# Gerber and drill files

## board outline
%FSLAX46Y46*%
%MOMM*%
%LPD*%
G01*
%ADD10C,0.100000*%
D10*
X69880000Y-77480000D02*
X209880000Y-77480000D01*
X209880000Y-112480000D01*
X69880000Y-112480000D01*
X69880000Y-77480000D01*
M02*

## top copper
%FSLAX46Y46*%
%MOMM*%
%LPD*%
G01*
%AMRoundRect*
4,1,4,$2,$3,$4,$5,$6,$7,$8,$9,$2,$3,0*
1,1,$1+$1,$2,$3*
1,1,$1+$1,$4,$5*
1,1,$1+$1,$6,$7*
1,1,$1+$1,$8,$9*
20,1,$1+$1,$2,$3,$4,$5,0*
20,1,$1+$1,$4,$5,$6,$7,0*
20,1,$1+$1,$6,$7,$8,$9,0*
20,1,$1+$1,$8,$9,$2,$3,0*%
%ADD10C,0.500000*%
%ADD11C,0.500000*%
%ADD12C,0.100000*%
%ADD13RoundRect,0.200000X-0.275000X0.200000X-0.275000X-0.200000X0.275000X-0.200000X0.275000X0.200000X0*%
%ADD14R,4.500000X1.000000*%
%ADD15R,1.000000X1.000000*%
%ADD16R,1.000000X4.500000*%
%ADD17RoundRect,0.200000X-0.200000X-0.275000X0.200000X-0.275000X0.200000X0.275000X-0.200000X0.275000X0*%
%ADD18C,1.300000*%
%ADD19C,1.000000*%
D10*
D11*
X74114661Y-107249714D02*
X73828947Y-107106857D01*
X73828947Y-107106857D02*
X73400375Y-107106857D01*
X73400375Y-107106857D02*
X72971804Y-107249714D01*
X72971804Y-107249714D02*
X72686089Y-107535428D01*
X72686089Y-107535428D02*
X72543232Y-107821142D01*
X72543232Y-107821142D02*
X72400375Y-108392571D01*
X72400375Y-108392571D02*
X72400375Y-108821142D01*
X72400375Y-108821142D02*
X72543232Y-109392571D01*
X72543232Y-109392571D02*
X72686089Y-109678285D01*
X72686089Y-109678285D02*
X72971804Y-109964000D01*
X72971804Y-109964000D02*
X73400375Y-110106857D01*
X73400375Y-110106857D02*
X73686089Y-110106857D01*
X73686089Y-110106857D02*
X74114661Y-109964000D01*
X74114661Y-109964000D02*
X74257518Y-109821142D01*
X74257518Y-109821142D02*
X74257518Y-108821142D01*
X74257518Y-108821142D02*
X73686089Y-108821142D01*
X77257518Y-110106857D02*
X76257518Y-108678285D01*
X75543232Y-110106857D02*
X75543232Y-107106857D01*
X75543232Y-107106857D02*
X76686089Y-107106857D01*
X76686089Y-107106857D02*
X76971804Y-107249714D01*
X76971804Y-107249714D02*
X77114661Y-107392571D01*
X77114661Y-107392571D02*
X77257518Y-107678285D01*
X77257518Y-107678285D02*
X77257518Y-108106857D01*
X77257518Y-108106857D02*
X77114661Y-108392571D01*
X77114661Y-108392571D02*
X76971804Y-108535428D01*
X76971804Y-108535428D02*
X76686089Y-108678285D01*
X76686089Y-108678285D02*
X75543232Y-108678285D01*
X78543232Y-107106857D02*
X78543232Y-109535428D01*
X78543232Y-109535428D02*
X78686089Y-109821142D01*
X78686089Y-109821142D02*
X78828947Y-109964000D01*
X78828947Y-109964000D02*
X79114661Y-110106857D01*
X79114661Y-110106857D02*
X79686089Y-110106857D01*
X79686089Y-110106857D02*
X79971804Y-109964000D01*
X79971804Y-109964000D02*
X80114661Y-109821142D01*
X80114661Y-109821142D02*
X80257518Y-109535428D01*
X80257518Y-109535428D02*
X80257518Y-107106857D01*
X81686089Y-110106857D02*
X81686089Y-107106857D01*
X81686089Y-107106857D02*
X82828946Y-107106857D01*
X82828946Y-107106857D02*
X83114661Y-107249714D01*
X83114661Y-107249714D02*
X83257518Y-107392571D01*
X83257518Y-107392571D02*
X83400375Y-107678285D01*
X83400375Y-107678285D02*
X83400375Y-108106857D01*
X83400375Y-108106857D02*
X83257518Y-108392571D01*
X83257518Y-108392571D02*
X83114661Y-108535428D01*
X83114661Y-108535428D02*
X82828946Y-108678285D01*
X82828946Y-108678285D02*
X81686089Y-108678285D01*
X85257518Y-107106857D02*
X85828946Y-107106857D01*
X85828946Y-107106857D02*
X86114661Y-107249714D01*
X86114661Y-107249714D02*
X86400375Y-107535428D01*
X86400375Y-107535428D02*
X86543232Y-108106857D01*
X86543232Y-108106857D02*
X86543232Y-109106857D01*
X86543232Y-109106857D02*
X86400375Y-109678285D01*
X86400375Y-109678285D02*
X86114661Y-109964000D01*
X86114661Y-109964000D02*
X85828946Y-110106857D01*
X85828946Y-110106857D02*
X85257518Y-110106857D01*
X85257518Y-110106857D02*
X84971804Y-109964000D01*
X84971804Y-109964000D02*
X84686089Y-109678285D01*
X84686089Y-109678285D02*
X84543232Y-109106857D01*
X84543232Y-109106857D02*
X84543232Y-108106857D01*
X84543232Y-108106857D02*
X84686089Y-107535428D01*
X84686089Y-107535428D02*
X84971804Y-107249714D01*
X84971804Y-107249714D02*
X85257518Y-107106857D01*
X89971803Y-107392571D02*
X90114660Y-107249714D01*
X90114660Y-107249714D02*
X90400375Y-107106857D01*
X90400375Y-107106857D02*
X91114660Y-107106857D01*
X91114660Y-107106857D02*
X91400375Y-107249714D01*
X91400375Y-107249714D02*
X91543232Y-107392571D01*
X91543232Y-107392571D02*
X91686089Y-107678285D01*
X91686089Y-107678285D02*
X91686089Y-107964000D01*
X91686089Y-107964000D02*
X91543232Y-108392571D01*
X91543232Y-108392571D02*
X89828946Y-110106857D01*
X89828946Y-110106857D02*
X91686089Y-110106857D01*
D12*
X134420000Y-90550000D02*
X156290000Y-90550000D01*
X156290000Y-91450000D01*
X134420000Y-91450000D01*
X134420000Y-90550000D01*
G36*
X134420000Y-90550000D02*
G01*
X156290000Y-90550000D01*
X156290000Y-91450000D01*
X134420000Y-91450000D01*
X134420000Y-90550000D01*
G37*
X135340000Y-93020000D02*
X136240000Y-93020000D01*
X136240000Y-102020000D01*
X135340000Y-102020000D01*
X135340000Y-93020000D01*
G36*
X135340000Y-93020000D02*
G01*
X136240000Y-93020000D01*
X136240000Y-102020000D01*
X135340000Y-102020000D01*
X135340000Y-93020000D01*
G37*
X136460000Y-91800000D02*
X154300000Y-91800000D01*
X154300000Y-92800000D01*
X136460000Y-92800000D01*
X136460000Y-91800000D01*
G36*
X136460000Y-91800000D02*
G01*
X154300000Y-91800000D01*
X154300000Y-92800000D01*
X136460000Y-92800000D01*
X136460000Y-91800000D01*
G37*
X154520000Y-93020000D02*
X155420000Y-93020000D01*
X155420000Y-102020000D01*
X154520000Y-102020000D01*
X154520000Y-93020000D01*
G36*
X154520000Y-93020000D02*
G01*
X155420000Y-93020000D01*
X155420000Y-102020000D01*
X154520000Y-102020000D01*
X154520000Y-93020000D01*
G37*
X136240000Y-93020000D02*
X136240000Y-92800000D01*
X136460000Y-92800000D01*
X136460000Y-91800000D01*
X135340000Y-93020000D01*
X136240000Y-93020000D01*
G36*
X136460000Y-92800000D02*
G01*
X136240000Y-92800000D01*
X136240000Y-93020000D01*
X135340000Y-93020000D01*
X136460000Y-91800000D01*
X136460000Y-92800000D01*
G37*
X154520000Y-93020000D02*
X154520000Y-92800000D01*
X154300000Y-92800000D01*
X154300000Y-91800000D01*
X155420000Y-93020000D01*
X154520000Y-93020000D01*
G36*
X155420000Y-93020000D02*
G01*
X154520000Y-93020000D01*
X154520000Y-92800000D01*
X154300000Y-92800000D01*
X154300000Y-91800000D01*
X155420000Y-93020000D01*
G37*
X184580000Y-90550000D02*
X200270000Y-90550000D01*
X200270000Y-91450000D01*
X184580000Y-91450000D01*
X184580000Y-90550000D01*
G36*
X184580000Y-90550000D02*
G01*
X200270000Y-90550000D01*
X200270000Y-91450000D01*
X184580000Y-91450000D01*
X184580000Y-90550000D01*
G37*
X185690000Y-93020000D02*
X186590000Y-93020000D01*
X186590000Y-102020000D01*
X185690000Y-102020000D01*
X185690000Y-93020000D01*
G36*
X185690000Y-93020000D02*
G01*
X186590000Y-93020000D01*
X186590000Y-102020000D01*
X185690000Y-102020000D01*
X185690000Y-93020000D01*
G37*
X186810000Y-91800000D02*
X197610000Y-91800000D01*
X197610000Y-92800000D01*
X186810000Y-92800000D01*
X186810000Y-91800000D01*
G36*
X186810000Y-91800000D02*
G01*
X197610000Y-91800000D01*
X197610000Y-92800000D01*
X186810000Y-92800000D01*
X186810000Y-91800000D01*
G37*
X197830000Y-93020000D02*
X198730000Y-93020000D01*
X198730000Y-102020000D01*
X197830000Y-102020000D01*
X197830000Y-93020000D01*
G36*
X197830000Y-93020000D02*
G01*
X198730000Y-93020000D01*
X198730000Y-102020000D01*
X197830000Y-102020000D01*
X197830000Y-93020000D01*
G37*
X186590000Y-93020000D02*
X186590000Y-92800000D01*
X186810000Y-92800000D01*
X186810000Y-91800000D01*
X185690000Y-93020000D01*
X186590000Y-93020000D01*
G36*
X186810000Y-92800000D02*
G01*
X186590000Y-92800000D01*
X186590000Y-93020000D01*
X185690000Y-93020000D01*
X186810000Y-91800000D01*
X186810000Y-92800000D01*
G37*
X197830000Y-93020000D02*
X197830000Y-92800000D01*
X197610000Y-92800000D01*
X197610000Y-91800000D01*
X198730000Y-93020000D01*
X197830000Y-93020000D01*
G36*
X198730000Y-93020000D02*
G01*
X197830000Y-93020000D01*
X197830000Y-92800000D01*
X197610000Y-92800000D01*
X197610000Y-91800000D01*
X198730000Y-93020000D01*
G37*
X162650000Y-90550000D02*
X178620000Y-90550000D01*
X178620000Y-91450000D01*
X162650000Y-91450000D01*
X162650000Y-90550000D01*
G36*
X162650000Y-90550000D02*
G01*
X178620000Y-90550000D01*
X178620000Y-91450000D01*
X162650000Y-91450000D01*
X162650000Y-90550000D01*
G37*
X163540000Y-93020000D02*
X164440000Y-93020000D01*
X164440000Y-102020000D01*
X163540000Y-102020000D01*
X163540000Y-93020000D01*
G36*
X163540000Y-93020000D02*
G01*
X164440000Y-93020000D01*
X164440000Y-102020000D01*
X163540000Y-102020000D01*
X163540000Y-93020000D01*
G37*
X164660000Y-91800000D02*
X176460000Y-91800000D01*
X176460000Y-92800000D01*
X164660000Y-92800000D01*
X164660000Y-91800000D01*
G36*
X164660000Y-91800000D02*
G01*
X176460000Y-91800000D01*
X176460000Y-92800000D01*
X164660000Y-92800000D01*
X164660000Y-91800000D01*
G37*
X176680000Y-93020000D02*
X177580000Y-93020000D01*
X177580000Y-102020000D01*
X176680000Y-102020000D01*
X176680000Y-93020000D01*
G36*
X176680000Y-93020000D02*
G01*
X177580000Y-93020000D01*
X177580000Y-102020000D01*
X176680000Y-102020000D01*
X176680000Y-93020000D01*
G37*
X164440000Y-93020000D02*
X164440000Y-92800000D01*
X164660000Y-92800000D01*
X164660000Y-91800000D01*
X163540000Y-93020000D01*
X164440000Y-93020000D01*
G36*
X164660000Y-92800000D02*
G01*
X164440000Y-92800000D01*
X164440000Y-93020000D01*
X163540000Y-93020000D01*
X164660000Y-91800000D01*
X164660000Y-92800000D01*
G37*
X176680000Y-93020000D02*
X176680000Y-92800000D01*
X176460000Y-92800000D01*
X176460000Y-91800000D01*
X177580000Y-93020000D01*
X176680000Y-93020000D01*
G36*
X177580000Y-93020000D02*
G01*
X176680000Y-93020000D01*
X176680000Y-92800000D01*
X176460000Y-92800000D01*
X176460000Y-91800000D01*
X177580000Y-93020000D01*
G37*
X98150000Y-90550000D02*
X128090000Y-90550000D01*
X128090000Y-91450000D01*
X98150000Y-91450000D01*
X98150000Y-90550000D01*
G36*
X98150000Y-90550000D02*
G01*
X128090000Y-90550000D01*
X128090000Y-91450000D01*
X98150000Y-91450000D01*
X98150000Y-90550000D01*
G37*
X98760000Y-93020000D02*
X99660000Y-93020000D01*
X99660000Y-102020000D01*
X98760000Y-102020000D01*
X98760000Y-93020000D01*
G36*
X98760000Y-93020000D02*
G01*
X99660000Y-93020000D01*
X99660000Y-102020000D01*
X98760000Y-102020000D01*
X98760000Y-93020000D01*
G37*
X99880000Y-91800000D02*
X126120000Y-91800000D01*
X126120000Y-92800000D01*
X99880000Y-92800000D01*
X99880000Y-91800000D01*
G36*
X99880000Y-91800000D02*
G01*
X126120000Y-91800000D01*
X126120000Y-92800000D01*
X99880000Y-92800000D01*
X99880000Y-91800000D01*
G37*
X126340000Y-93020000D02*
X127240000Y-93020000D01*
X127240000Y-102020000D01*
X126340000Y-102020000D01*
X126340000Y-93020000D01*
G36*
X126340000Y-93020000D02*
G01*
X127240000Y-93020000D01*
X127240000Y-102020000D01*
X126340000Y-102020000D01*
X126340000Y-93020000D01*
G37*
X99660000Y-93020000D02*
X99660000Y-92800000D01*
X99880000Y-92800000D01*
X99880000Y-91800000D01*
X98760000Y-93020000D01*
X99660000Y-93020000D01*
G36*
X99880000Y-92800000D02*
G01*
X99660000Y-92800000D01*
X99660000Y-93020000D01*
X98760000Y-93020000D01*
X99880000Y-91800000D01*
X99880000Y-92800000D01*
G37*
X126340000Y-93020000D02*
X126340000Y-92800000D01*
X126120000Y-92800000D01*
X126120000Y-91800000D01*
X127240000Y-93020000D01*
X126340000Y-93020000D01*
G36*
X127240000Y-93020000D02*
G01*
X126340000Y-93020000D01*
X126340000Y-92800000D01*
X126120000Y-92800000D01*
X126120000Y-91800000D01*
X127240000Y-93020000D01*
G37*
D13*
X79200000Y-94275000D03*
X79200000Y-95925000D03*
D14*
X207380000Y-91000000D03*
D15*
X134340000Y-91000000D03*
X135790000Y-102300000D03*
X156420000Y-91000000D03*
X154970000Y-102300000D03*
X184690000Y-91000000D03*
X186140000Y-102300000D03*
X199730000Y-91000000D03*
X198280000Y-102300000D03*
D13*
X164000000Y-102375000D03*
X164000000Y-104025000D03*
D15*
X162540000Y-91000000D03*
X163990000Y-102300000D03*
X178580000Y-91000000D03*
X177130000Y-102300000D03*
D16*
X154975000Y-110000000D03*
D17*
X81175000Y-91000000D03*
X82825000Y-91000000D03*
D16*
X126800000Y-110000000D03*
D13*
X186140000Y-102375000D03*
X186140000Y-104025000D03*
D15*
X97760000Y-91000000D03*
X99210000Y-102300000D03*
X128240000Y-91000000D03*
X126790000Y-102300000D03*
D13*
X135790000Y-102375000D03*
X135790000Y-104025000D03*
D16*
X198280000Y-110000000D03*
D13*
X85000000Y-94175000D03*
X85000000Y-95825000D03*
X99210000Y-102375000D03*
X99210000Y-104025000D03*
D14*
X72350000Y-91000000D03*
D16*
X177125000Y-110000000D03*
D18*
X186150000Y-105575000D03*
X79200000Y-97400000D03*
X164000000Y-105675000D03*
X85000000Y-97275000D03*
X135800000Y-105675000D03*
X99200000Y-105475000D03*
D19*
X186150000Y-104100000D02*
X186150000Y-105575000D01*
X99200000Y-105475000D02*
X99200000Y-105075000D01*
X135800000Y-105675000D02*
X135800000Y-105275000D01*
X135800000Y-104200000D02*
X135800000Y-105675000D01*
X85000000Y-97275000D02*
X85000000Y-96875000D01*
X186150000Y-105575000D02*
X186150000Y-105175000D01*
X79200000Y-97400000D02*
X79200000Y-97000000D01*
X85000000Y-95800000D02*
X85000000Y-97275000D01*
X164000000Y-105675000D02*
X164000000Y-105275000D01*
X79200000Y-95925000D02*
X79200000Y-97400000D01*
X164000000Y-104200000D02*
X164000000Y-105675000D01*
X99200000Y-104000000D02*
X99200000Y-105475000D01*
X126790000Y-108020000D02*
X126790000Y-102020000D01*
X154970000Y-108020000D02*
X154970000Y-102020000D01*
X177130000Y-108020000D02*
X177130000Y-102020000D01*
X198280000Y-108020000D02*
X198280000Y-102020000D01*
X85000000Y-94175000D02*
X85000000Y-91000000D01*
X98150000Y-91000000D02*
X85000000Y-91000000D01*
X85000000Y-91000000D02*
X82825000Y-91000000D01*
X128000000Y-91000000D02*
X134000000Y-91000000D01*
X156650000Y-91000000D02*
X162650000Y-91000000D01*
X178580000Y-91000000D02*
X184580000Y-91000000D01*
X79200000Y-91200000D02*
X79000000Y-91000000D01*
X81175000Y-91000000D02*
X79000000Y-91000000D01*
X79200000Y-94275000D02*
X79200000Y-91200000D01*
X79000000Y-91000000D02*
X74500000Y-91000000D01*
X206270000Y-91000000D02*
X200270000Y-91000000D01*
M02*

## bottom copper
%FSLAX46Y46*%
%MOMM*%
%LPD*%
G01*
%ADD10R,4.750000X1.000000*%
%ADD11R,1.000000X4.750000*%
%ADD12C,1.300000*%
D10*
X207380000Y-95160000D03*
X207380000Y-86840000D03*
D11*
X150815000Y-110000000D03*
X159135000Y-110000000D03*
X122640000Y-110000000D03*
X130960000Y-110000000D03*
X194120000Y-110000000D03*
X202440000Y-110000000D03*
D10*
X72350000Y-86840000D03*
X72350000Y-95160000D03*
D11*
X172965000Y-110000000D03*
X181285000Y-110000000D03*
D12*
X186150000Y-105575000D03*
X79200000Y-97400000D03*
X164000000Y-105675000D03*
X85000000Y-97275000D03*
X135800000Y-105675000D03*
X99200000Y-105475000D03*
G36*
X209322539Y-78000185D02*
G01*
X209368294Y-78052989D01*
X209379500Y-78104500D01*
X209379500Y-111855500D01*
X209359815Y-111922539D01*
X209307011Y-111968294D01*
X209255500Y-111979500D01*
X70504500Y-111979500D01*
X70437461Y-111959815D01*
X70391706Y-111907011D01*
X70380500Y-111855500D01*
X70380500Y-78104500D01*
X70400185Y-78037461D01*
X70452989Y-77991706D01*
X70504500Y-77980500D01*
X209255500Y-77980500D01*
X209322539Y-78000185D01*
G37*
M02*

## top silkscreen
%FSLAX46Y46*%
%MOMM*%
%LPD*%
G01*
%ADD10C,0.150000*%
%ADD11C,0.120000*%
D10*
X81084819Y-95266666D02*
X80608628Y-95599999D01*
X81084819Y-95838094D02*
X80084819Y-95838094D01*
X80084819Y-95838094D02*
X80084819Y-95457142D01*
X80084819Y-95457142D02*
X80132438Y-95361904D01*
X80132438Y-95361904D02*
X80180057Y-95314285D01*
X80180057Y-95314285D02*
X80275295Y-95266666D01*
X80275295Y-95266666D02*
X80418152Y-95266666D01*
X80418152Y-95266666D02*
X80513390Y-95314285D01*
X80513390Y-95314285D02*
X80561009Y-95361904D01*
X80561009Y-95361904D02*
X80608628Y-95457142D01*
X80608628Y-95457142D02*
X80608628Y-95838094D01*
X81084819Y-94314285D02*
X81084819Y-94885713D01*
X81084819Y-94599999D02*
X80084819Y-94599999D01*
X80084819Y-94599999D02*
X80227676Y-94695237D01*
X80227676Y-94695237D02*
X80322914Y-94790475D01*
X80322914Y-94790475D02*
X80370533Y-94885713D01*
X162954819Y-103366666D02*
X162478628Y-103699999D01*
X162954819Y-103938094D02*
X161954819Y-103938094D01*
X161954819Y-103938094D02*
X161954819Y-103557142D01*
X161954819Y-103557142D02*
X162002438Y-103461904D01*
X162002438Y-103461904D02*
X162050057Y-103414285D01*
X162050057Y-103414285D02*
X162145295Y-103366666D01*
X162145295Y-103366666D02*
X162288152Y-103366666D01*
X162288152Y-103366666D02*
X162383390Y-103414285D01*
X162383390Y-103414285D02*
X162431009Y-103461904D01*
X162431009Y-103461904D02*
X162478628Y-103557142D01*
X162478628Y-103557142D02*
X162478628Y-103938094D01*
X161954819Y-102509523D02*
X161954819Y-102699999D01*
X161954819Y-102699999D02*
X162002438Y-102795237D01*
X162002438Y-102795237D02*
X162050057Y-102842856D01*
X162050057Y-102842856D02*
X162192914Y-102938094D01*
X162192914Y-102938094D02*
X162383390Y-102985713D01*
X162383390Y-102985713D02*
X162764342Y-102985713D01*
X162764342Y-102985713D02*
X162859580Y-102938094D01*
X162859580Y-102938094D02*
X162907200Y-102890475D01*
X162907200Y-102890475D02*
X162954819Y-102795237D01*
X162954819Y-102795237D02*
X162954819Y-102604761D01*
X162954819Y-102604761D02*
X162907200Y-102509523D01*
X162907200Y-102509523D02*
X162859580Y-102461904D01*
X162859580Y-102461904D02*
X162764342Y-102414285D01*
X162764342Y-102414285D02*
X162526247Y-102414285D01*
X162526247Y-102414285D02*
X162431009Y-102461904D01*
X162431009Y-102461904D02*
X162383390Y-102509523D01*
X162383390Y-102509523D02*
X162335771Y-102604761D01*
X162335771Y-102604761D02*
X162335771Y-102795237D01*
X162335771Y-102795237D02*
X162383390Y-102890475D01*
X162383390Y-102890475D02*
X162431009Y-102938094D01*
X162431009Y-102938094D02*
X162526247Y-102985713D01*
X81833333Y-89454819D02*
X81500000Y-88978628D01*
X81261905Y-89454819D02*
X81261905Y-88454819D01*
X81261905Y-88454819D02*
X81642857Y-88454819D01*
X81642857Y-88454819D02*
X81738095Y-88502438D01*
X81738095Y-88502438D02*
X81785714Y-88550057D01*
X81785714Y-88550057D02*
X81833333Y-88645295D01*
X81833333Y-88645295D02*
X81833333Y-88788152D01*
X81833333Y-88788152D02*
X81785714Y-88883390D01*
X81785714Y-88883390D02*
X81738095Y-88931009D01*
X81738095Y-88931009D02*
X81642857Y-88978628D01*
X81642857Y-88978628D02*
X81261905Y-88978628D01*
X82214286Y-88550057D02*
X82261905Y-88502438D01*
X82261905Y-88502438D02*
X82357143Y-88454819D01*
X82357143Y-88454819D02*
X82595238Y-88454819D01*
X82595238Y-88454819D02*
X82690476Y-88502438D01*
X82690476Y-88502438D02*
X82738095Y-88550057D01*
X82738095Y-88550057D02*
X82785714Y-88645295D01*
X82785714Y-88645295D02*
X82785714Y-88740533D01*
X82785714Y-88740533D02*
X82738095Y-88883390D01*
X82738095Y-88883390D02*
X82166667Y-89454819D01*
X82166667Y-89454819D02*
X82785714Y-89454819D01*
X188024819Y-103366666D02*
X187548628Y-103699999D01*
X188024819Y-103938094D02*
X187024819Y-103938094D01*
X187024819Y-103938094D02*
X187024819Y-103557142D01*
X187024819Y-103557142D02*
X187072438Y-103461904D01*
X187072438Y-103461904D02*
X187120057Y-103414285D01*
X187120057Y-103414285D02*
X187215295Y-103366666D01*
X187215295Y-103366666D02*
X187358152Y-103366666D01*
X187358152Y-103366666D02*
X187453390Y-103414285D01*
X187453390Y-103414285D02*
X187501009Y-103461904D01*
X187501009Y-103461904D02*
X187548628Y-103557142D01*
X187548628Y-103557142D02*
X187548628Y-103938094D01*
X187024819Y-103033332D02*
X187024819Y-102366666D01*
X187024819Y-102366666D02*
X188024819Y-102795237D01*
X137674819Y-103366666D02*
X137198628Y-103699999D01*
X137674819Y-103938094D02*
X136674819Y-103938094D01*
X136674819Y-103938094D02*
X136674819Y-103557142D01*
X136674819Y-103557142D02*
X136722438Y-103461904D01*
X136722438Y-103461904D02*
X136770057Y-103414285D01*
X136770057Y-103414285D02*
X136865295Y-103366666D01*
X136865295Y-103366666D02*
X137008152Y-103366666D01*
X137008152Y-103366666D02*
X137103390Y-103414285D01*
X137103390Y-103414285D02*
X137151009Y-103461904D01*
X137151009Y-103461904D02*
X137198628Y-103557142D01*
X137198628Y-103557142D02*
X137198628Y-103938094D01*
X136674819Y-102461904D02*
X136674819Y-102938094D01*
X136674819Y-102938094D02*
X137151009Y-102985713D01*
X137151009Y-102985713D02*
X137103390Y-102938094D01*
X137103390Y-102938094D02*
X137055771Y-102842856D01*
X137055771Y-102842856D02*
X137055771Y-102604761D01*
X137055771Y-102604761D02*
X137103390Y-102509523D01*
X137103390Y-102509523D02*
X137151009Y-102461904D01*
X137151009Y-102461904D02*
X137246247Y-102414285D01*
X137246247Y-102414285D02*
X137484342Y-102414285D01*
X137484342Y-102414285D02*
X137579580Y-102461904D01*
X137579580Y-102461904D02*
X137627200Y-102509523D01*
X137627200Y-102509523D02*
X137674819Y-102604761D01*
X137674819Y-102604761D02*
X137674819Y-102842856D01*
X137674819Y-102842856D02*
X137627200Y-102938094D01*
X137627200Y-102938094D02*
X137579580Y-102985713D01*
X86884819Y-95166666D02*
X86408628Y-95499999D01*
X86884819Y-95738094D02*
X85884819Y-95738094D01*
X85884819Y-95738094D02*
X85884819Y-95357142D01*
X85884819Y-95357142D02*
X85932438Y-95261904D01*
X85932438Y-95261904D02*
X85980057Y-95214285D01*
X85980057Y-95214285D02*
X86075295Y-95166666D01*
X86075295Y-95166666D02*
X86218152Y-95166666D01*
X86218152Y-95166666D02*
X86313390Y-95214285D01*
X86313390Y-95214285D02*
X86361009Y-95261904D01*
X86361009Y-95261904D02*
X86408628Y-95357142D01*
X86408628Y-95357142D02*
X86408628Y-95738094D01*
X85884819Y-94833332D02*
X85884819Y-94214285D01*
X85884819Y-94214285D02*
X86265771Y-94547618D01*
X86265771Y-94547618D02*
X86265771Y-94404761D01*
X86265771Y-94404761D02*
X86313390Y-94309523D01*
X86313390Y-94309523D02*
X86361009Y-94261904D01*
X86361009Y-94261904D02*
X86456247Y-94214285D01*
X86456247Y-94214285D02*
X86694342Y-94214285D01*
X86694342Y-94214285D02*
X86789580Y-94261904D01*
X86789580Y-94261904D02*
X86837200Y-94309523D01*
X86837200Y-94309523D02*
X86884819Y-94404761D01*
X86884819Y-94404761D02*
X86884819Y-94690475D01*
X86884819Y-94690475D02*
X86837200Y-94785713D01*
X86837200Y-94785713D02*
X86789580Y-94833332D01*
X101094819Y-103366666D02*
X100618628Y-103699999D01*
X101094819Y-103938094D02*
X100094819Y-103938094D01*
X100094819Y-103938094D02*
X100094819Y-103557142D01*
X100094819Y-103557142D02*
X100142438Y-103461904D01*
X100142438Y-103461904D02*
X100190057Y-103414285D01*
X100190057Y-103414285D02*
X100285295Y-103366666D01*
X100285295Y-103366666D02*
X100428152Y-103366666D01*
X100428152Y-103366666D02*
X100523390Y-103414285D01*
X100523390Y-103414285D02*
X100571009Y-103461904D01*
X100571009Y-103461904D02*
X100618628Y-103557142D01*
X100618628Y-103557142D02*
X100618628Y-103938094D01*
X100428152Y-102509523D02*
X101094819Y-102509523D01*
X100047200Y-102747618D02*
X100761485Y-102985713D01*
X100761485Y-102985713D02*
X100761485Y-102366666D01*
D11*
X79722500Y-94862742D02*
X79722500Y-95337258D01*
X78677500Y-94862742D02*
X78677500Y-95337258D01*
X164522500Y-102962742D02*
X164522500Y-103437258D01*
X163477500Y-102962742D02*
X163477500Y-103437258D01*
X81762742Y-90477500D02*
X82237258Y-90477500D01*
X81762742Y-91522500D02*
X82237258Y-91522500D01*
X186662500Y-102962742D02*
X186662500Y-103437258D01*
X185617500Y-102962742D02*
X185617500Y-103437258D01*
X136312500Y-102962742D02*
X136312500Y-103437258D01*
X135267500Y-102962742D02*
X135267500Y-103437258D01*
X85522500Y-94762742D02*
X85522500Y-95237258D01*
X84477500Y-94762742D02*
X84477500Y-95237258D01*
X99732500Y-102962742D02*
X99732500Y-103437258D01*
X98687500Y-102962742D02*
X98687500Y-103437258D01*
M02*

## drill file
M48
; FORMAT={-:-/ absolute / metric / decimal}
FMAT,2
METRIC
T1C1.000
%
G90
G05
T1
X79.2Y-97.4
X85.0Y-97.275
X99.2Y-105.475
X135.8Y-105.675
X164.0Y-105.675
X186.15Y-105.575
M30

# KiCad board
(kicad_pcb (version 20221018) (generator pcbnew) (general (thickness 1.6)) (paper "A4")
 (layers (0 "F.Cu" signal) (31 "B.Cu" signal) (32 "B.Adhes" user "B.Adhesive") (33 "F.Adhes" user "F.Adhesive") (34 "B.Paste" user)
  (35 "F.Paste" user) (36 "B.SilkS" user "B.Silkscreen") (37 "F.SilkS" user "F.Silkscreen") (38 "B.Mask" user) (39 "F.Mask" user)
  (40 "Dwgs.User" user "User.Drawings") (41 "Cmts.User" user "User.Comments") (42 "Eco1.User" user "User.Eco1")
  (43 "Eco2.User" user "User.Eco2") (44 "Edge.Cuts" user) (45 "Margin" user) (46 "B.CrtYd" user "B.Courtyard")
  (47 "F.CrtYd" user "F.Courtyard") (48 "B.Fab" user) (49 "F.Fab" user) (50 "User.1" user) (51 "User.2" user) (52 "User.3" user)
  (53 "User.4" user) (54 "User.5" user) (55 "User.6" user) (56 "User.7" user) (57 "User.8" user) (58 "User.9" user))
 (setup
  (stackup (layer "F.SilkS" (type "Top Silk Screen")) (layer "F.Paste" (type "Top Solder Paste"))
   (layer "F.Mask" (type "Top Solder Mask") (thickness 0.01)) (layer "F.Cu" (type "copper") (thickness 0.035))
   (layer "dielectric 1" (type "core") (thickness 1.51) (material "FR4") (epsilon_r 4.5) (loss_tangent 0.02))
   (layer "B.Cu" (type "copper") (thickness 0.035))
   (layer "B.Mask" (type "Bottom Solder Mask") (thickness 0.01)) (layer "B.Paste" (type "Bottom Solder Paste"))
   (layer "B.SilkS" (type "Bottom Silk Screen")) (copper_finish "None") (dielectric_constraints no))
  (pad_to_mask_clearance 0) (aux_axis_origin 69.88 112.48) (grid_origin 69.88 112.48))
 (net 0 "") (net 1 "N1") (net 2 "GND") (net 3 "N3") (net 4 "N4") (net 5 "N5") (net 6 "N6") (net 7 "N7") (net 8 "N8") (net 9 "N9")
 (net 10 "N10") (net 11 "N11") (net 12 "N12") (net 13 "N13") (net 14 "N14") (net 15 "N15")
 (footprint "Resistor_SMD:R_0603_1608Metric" (layer "F.Cu") (at 79.2 95.1 -90)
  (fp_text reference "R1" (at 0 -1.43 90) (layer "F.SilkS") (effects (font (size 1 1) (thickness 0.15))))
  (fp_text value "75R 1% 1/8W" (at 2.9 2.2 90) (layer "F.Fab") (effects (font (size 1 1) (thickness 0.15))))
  (fp_line (start -0.237258 -0.5225) (end 0.237258 -0.5225) (stroke (width 0.12) (type solid)) (layer "F.SilkS"))
  (fp_line (start -0.237258 0.5225) (end 0.237258 0.5225) (stroke (width 0.12) (type solid)) (layer "F.SilkS"))
  (pad "1" smd roundrect (at -0.825 0 270) (size 0.8 0.95) (layers "F.Cu" "F.Paste" "F.Mask") (roundrect_rratio 0.25) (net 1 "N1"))
  (pad "2" smd roundrect (at 0.825 0 270) (size 0.8 0.95) (layers "F.Cu" "F.Paste" "F.Mask") (roundrect_rratio 0.25) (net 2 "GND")))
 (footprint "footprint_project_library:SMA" (layer "F.Cu") (at 207.38 91 180)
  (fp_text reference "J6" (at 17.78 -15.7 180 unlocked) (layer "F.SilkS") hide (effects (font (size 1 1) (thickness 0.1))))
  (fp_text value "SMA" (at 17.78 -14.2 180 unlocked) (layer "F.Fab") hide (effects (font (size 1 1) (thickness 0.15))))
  (pad "1" smd rect (at 0 0 180) (size 4.5 1) (layers "F.Cu") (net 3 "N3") (thermal_bridge_angle 45))
  (pad "2" smd rect (at 0 -4.16 180) (size 4.75 1) (layers "B.Cu") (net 2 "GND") (thermal_bridge_angle 45))
  (pad "2" smd rect (at 0 4.16 180) (size 4.75 1) (layers "B.Cu") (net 2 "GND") (thermal_bridge_angle 45)))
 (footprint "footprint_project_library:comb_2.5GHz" (layer "F.Cu") (at 145.38 91)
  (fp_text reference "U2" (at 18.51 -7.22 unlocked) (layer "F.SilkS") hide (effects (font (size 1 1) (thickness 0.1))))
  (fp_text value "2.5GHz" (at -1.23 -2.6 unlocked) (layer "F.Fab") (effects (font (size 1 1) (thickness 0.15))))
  (fp_rect (start -10.96 -0.45) (end 10.91 0.45) (stroke (width 0.1) (type solid)) (fill solid) (layer "F.Cu"))
  (fp_rect (start -10.04 2.02) (end -9.14 11.02) (stroke (width 0.1) (type solid)) (fill solid) (layer "F.Cu"))
  (fp_rect (start -8.92 0.8) (end 8.92 1.8) (stroke (width 0.1) (type solid)) (fill solid) (layer "F.Cu"))
  (fp_rect (start 10.04 2.02) (end 9.14 11.02) (stroke (width 0.1) (type solid)) (fill solid) (layer "F.Cu"))
  (fp_poly
   (pts (xy -9.14 2.02) (xy -9.14 1.8) (xy -8.92 1.8) (xy -8.92 0.8) (xy -10.04 2.02)) (stroke (width 0.1) (type solid)) (fill solid)
   (layer "F.Cu"))
  (fp_poly
   (pts (xy 9.14 2.02) (xy 9.14 1.8) (xy 8.92 1.8) (xy 8.92 0.8) (xy 10.04 2.02)) (stroke (width 0.1) (type solid)) (fill solid)
   (layer "F.Cu"))
  (pad "1" smd rect (at -11.04 0) (size 1 1) (layers "F.Cu") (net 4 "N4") (thermal_bridge_angle 45))
  (pad "2" smd rect (at -9.59 11.3) (size 1 1) (layers "F.Cu") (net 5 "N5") (thermal_bridge_angle 45))
  (pad "3" smd rect (at 11.04 0) (size 1 1) (layers "F.Cu") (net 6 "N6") (thermal_bridge_angle 45))
  (pad "4" smd rect (at 9.59 11.3) (size 1 1) (layers "F.Cu") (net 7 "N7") (thermal_bridge_angle 45)))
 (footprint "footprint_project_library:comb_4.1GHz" (layer "F.Cu") (at 192.21 91)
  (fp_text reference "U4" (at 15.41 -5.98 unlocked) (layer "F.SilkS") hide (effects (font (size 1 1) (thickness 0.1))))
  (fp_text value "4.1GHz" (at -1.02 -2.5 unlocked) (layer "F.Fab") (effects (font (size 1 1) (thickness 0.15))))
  (fp_rect (start -7.63 -0.45) (end 8.06 0.45) (stroke (width 0.1) (type solid)) (fill solid) (layer "F.Cu"))
  (fp_rect (start -6.52 2.02) (end -5.62 11.02) (stroke (width 0.1) (type solid)) (fill solid) (layer "F.Cu"))
  (fp_rect (start -5.4 0.8) (end 5.4 1.8) (stroke (width 0.1) (type solid)) (fill solid) (layer "F.Cu"))
  (fp_rect (start 6.52 2.02) (end 5.62 11.02) (stroke (width 0.1) (type solid)) (fill solid) (layer "F.Cu"))
  (fp_poly
   (pts (xy -5.62 2.02) (xy -5.62 1.8) (xy -5.4 1.8) (xy -5.4 0.8) (xy -6.52 2.02)) (stroke (width 0.1) (type solid)) (fill solid)
   (layer "F.Cu"))
  (fp_poly
   (pts (xy 5.62 2.02) (xy 5.62 1.8) (xy 5.4 1.8) (xy 5.4 0.8) (xy 6.52 2.02)) (stroke (width 0.1) (type solid)) (fill solid) (layer "F.Cu"))
  (pad "1" smd rect (at -7.52 0) (size 1 1) (layers "F.Cu") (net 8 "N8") (thermal_bridge_angle 45))
  (pad "2" smd rect (at -6.07 11.3) (size 1 1) (layers "F.Cu") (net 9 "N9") (thermal_bridge_angle 45))
  (pad "3" smd rect (at 7.52 0) (size 1 1) (layers "F.Cu") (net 3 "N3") (thermal_bridge_angle 45))
  (pad "4" smd rect (at 6.07 11.3) (size 1 1) (layers "F.Cu") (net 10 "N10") (thermal_bridge_angle 45)))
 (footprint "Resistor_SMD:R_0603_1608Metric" (layer "F.Cu") (at 164 103.2 -90)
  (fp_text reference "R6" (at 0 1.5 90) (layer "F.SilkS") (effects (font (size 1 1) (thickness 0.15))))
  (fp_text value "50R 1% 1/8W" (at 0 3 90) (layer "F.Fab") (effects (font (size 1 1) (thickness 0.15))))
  (fp_line (start -0.237258 -0.5225) (end 0.237258 -0.5225) (stroke (width 0.12) (type solid)) (layer "F.SilkS"))
  (fp_line (start -0.237258 0.5225) (end 0.237258 0.5225) (stroke (width 0.12) (type solid)) (layer "F.SilkS"))
  (pad "1" smd roundrect (at -0.825 0 270) (size 0.8 0.95) (layers "F.Cu" "F.Paste" "F.Mask") (roundrect_rratio 0.25) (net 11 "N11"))
  (pad "2" smd roundrect (at 0.825 0 270) (size 0.8 0.95) (layers "F.Cu" "F.Paste" "F.Mask") (roundrect_rratio 0.25) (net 2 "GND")))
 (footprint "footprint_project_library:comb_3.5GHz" (layer "F.Cu") (at 170.56 91)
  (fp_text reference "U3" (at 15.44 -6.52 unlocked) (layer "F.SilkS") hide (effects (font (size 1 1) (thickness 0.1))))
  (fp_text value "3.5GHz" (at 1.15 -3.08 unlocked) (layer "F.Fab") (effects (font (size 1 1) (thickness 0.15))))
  (fp_rect (start -7.91 -0.45) (end 8.06 0.45) (stroke (width 0.1) (type solid)) (fill solid) (layer "F.Cu"))
  (fp_rect (start -7.02 2.02) (end -6.12 11.02) (stroke (width 0.1) (type solid)) (fill solid) (layer "F.Cu"))
  (fp_rect (start -5.9 0.8) (end 5.9 1.8) (stroke (width 0.1) (type solid)) (fill solid) (layer "F.Cu"))
  (fp_rect (start 7.02 2.02) (end 6.12 11.02) (stroke (width 0.1) (type solid)) (fill solid) (layer "F.Cu"))
  (fp_poly
   (pts (xy -6.12 2.02) (xy -6.12 1.8) (xy -5.9 1.8) (xy -5.9 0.8) (xy -7.02 2.02)) (stroke (width 0.1) (type solid)) (fill solid)
   (layer "F.Cu"))
  (fp_poly
   (pts (xy 6.12 2.02) (xy 6.12 1.8) (xy 5.9 1.8) (xy 5.9 0.8) (xy 7.02 2.02)) (stroke (width 0.1) (type solid)) (fill solid) (layer "F.Cu"))
  (pad "1" smd rect (at -8.02 0) (size 1 1) (layers "F.Cu") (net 6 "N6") (thermal_bridge_angle 45))
  (pad "2" smd rect (at -6.57 11.3) (size 1 1) (layers "F.Cu") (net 11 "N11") (thermal_bridge_angle 45))
  (pad "3" smd rect (at 8.02 0) (size 1 1) (layers "F.Cu") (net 8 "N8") (thermal_bridge_angle 45))
  (pad "4" smd rect (at 6.57 11.3) (size 1 1) (layers "F.Cu") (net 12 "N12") (thermal_bridge_angle 45)))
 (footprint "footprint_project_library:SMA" (layer "F.Cu") (at 154.975 110 90)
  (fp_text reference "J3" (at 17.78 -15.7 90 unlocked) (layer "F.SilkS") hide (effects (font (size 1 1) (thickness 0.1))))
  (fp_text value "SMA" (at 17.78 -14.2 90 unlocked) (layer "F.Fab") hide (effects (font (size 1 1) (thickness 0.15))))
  (pad "1" smd rect (at 0 0 90) (size 4.5 1) (layers "F.Cu") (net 7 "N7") (thermal_bridge_angle 45))
  (pad "2" smd rect (at 0 -4.16 90) (size 4.75 1) (layers "B.Cu") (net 2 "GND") (thermal_bridge_angle 45))
  (pad "2" smd rect (at 0 4.16 90) (size 4.75 1) (layers "B.Cu") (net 2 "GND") (thermal_bridge_angle 45)))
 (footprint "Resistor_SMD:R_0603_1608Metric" (layer "F.Cu") (at 82 91)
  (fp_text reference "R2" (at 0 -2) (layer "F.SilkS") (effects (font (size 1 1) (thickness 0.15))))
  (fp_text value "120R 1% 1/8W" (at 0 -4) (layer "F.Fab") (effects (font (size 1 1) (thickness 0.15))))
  (fp_line (start -0.237258 -0.5225) (end 0.237258 -0.5225) (stroke (width 0.12) (type solid)) (layer "F.SilkS"))
  (fp_line (start -0.237258 0.5225) (end 0.237258 0.5225) (stroke (width 0.12) (type solid)) (layer "F.SilkS"))
  (pad "1" smd roundrect (at -0.825 0) (size 0.8 0.95) (layers "F.Cu" "F.Paste" "F.Mask") (roundrect_rratio 0.25) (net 1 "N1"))
  (pad "2" smd roundrect (at 0.825 0) (size 0.8 0.95) (layers "F.Cu" "F.Paste" "F.Mask") (roundrect_rratio 0.25) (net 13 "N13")))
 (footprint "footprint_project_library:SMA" (layer "F.Cu") (at 126.8 110 90)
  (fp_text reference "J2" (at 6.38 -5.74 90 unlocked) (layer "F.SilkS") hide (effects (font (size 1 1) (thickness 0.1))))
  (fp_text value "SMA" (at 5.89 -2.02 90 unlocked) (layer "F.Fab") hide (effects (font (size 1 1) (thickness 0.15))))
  (pad "1" smd rect (at 0 0 90) (size 4.5 1) (layers "F.Cu") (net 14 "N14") (thermal_bridge_angle 45))
  (pad "2" smd rect (at 0 -4.16 90) (size 4.75 1) (layers "B.Cu") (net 2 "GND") (thermal_bridge_angle 45))
  (pad "2" smd rect (at 0 4.16 90) (size 4.75 1) (layers "B.Cu") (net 2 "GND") (thermal_bridge_angle 45)))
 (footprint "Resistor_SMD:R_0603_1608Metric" (layer "F.Cu") (at 186.14 103.2 -90)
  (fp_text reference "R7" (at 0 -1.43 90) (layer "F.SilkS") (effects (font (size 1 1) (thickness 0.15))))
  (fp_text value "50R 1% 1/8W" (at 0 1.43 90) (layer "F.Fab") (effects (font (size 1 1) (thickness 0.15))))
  (fp_line (start -0.237258 -0.5225) (end 0.237258 -0.5225) (stroke (width 0.12) (type solid)) (layer "F.SilkS"))
  (fp_line (start -0.237258 0.5225) (end 0.237258 0.5225) (stroke (width 0.12) (type solid)) (layer "F.SilkS"))
  (pad "1" smd roundrect (at -0.825 0 270) (size 0.8 0.95) (layers "F.Cu" "F.Paste" "F.Mask") (roundrect_rratio 0.25) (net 9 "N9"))
  (pad "2" smd roundrect (at 0.825 0 270) (size 0.8 0.95) (layers "F.Cu" "F.Paste" "F.Mask") (roundrect_rratio 0.25) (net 2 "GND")))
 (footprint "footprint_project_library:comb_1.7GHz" (layer "F.Cu") (at 113 91)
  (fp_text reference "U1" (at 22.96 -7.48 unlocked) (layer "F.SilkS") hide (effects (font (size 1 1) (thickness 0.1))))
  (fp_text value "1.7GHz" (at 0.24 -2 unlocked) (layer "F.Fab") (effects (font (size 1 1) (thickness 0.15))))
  (fp_rect (start -14.85 -0.45) (end 15.09 0.45) (stroke (width 0.1) (type solid)) (fill solid) (layer "F.Cu"))
  (fp_rect (start -14.24 2.02) (end -13.34 11.02) (stroke (width 0.1) (type solid)) (fill solid) (layer "F.Cu"))
  (fp_rect (start -13.12 0.8) (end 13.12 1.8) (stroke (width 0.1) (type solid)) (fill solid) (layer "F.Cu"))
  (fp_rect (start 14.24 2.02) (end 13.34 11.02) (stroke (width 0.1) (type solid)) (fill solid) (layer "F.Cu"))
  (fp_poly
   (pts (xy -13.34 2.02) (xy -13.34 1.8) (xy -13.12 1.8) (xy -13.12 0.8) (xy -14.24 2.02)) (stroke (width 0.1) (type solid)) (fill solid)
   (layer "F.Cu"))
  (fp_poly
   (pts (xy 13.34 2.02) (xy 13.34 1.8) (xy 13.12 1.8) (xy 13.12 0.8) (xy 14.24 2.02)) (stroke (width 0.1) (type solid)) (fill solid)
   (layer "F.Cu"))
  (pad "1" smd rect (at -15.24 0) (size 1 1) (layers "F.Cu") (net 13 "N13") (thermal_bridge_angle 45))
  (pad "2" smd rect (at -13.79 11.3) (size 1 1) (layers "F.Cu") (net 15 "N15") (thermal_bridge_angle 45))
  (pad "3" smd rect (at 15.24 0) (size 1 1) (layers "F.Cu") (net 4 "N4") (thermal_bridge_angle 45))
  (pad "4" smd rect (at 13.79 11.3) (size 1 1) (layers "F.Cu") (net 14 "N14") (thermal_bridge_angle 45)))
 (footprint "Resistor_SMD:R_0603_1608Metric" (layer "F.Cu") (at 135.79 103.2 -90)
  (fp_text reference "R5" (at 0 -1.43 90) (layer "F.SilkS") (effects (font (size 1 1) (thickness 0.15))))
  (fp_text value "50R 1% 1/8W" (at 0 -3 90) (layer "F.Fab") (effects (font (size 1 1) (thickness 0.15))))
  (fp_line (start -0.237258 -0.5225) (end 0.237258 -0.5225) (stroke (width 0.12) (type solid)) (layer "F.SilkS"))
  (fp_line (start -0.237258 0.5225) (end 0.237258 0.5225) (stroke (width 0.12) (type solid)) (layer "F.SilkS"))
  (pad "1" smd roundrect (at -0.825 0 270) (size 0.8 0.95) (layers "F.Cu" "F.Paste" "F.Mask") (roundrect_rratio 0.25) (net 5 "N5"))
  (pad "2" smd roundrect (at 0.825 0 270) (size 0.8 0.95) (layers "F.Cu" "F.Paste" "F.Mask") (roundrect_rratio 0.25) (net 2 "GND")))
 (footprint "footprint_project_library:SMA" (layer "F.Cu") (at 198.28 110 90)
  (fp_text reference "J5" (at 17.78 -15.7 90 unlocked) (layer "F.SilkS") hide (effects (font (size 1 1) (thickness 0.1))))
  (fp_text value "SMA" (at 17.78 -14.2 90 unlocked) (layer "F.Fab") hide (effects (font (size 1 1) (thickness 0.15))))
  (pad "1" smd rect (at 0 0 90) (size 4.5 1) (layers "F.Cu") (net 10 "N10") (thermal_bridge_angle 45))
  (pad "2" smd rect (at 0 -4.16 90) (size 4.75 1) (layers "B.Cu") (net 2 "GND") (thermal_bridge_angle 45))
  (pad "2" smd rect (at 0 4.16 90) (size 4.75 1) (layers "B.Cu") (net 2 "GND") (thermal_bridge_angle 45)))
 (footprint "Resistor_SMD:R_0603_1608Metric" (layer "F.Cu") (at 85 95 -90)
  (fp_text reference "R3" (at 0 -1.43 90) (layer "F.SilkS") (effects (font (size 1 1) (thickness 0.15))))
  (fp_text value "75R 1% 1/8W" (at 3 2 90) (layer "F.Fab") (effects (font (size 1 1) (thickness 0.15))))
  (fp_line (start -0.237258 -0.5225) (end 0.237258 -0.5225) (stroke (width 0.12) (type solid)) (layer "F.SilkS"))
  (fp_line (start -0.237258 0.5225) (end 0.237258 0.5225) (stroke (width 0.12) (type solid)) (layer "F.SilkS"))
  (pad "1" smd roundrect (at -0.825 0 270) (size 0.8 0.95) (layers "F.Cu" "F.Paste" "F.Mask") (roundrect_rratio 0.25) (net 13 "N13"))
  (pad "2" smd roundrect (at 0.825 0 270) (size 0.8 0.95) (layers "F.Cu" "F.Paste" "F.Mask") (roundrect_rratio 0.25) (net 2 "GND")))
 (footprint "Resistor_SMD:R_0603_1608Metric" (layer "F.Cu") (at 99.21 103.2 -90)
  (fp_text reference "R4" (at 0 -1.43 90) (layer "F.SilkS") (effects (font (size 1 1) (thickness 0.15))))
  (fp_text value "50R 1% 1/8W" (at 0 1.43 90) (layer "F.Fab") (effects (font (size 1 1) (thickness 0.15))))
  (fp_line (start -0.237258 -0.5225) (end 0.237258 -0.5225) (stroke (width 0.12) (type solid)) (layer "F.SilkS"))
  (fp_line (start -0.237258 0.5225) (end 0.237258 0.5225) (stroke (width 0.12) (type solid)) (layer "F.SilkS"))
  (pad "1" smd roundrect (at -0.825 0 270) (size 0.8 0.95) (layers "F.Cu" "F.Paste" "F.Mask") (roundrect_rratio 0.25) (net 15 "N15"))
  (pad "2" smd roundrect (at 0.825 0 270) (size 0.8 0.95) (layers "F.Cu" "F.Paste" "F.Mask") (roundrect_rratio 0.25) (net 2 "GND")))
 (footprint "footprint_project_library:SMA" (layer "F.Cu") (at 72.35 91)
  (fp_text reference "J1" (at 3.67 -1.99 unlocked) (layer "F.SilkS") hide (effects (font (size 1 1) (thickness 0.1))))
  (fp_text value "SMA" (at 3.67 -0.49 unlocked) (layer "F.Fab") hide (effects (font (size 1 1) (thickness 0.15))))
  (pad "1" smd rect (at 0 0) (size 4.5 1) (layers "F.Cu") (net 1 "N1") (thermal_bridge_angle 45))
  (pad "2" smd rect (at 0 -4.16) (size 4.75 1) (layers "B.Cu") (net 2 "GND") (thermal_bridge_angle 45))
  (pad "2" smd rect (at 0 4.16) (size 4.75 1) (layers "B.Cu") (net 2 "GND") (thermal_bridge_angle 45)))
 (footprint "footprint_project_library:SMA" (layer "F.Cu") (at 177.125 110 90)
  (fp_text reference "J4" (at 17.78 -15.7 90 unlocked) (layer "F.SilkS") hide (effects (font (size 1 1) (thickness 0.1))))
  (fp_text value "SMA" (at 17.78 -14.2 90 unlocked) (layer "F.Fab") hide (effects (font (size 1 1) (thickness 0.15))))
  (pad "1" smd rect (at 0 0 90) (size 4.5 1) (layers "F.Cu") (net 12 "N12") (thermal_bridge_angle 45))
  (pad "2" smd rect (at 0 -4.16 90) (size 4.75 1) (layers "B.Cu") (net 2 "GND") (thermal_bridge_angle 45))
  (pad "2" smd rect (at 0 4.16 90) (size 4.75 1) (layers "B.Cu") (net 2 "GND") (thermal_bridge_angle 45)))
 (gr_rect (start 69.88 77.48) (end 209.88 112.48) (stroke (width 0.1) (type default)) (fill none) (layer "Edge.Cuts"))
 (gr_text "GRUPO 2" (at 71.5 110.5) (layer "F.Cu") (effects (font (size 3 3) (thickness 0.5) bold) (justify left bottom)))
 (segment (start 186.15 104.1) (end 186.15 105.575) (width 1) (layer "F.Cu") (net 2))
 (segment (start 99.2 105.475) (end 99.2 105.075) (width 1) (layer "F.Cu") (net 2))
 (segment (start 135.8 105.675) (end 135.8 105.275) (width 1) (layer "F.Cu") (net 2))
 (segment (start 135.8 104.2) (end 135.8 105.675) (width 1) (layer "F.Cu") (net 2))
 (segment (start 85 97.275) (end 85 96.875) (width 1) (layer "F.Cu") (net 2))
 (segment (start 186.15 105.575) (end 186.15 105.175) (width 1) (layer "F.Cu") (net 2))
 (segment (start 79.2 97.4) (end 79.2 97) (width 1) (layer "F.Cu") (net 2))
 (segment (start 85 95.8) (end 85 97.275) (width 1) (layer "F.Cu") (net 2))
 (segment (start 164 105.675) (end 164 105.275) (width 1) (layer "F.Cu") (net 2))
 (segment (start 79.2 95.925) (end 79.2 97.4) (width 1) (layer "F.Cu") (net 2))
 (segment (start 164 104.2) (end 164 105.675) (width 1) (layer "F.Cu") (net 2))
 (segment (start 99.2 104) (end 99.2 105.475) (width 1) (layer "F.Cu") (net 2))
 (via (at 186.15 105.575) (size 1.3) (drill 1) (layers "F.Cu" "B.Cu") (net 2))
 (via (at 79.2 97.4) (size 1.3) (drill 1) (layers "F.Cu" "B.Cu") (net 2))
 (via (at 164 105.675) (size 1.3) (drill 1) (layers "F.Cu" "B.Cu") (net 2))
 (via (at 85 97.275) (size 1.3) (drill 1) (layers "F.Cu" "B.Cu") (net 2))
 (via (at 135.8 105.675) (size 1.3) (drill 1) (layers "F.Cu" "B.Cu") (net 2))
 (via (at 99.2 105.475) (size 1.3) (drill 1) (layers "F.Cu" "B.Cu") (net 2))
 (segment (start 126.79 108.02) (end 126.79 102.02) (width 1) (layer "F.Cu") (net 14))
 (segment (start 154.97 108.02) (end 154.97 102.02) (width 1) (layer "F.Cu") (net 7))
 (segment (start 177.13 108.02) (end 177.13 102.02) (width 1) (layer "F.Cu") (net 12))
 (segment (start 198.28 108.02) (end 198.28 102.02) (width 1) (layer "F.Cu") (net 10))
 (segment (start 85 94.175) (end 85 91) (width 1) (layer "F.Cu") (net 13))
 (segment (start 98.15 91) (end 85 91) (width 1) (layer "F.Cu") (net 13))
 (segment (start 85 91) (end 82.825 91) (width 1) (layer "F.Cu") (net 13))
 (segment (start 128 91) (end 134 91) (width 1) (layer "F.Cu") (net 4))
 (segment (start 156.65 91) (end 162.65 91) (width 1) (layer "F.Cu") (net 6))
 (segment (start 178.58 91) (end 184.58 91) (width 1) (layer "F.Cu") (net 8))
 (segment (start 79.2 91.2) (end 79 91) (width 1) (layer "F.Cu") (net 1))
 (segment (start 81.175 91) (end 79 91) (width 1) (layer "F.Cu") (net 1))
 (segment (start 79.2 94.275) (end 79.2 91.2) (width 1) (layer "F.Cu") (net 1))
 (segment (start 79 91) (end 74.5 91) (width 1) (layer "F.Cu") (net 1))
 (segment (start 206.27 91) (end 200.27 91) (width 1) (layer "F.Cu") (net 3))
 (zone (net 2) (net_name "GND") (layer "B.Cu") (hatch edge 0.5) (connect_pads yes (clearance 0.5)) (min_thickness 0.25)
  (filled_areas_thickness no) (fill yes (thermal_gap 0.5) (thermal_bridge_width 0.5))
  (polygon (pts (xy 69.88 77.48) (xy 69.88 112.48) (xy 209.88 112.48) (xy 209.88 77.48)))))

